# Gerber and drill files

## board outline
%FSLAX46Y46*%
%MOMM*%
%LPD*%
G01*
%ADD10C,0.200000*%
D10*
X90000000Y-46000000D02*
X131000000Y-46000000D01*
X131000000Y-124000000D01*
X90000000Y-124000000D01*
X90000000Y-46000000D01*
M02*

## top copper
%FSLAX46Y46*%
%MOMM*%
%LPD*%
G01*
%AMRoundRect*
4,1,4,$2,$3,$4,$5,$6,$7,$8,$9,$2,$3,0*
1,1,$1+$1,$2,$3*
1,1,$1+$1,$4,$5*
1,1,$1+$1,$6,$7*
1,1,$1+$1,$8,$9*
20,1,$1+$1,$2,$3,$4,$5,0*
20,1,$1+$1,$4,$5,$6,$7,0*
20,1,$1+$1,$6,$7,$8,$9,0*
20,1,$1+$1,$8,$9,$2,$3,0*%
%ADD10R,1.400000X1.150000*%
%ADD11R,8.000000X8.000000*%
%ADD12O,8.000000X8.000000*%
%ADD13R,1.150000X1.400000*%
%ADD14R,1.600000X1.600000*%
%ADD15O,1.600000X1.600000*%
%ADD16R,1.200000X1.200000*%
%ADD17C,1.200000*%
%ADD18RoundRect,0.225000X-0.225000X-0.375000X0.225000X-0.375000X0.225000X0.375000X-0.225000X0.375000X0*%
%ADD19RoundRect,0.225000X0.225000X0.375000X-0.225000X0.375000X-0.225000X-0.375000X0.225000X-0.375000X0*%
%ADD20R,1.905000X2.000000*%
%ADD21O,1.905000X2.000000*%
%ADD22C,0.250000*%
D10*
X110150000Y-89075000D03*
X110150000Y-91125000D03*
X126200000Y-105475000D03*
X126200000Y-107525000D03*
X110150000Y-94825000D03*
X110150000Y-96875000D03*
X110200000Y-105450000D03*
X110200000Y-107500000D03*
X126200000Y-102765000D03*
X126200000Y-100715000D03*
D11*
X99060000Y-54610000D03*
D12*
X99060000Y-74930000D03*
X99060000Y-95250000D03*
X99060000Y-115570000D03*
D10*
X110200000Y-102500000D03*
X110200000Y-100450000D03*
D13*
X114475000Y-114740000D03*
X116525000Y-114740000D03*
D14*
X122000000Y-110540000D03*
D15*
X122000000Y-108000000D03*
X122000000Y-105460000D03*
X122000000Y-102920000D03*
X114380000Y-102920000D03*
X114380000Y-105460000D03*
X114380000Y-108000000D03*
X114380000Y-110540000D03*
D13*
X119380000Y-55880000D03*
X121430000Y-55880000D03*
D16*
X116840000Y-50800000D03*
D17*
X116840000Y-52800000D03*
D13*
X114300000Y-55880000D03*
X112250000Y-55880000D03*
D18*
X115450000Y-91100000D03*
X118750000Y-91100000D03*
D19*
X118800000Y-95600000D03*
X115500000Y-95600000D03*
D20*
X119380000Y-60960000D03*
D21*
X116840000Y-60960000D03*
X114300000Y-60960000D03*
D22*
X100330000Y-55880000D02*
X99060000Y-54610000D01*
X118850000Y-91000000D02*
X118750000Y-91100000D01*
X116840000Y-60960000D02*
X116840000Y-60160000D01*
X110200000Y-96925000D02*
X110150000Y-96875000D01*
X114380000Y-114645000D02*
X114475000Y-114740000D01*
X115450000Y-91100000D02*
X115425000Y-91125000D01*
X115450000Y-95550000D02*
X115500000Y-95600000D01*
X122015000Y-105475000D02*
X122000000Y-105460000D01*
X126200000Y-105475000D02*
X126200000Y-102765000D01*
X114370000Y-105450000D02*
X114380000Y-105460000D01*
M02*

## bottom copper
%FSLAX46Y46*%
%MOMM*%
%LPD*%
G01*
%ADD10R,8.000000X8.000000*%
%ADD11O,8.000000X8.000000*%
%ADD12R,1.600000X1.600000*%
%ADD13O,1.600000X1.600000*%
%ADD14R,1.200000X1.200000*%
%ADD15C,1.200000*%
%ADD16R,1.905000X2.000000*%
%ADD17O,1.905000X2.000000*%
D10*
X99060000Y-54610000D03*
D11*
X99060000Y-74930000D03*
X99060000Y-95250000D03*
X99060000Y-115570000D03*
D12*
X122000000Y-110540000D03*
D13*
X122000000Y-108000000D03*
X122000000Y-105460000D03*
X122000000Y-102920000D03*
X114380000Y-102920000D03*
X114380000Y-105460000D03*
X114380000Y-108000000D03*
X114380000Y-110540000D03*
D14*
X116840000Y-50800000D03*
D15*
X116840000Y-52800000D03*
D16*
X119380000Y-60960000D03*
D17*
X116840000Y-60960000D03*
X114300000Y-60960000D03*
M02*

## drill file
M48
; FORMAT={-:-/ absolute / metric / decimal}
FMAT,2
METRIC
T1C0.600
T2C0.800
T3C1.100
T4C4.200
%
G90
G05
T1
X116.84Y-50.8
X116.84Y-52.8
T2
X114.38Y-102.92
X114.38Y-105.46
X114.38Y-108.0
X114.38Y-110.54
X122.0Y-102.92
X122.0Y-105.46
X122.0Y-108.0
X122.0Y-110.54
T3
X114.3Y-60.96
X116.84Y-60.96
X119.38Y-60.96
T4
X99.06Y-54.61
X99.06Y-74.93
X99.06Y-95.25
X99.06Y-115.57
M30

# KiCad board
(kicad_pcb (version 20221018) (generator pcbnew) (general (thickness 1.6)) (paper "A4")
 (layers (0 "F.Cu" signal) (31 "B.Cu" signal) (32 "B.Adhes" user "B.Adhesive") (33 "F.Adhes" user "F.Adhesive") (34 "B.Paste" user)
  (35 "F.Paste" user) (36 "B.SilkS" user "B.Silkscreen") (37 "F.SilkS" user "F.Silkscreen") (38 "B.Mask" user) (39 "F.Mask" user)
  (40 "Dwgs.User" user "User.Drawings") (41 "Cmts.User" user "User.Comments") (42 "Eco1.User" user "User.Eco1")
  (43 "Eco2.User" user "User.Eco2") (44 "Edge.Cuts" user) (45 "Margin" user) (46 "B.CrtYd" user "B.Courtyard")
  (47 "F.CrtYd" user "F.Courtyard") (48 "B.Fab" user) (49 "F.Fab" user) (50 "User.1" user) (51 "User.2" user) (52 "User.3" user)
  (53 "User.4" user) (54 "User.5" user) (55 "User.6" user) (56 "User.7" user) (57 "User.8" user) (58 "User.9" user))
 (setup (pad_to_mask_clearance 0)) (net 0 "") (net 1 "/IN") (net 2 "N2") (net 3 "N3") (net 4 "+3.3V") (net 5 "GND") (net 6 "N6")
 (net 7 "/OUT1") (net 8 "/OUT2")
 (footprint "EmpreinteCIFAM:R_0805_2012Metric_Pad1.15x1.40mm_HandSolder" (layer "F.Cu") (at 110.15 90.1 -90)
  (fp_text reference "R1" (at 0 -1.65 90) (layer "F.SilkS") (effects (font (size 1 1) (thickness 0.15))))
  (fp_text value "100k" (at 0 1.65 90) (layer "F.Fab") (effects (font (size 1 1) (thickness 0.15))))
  (pad "1" smd rect (at -1.025 0 270) (size 1.15 1.4) (layers "F.Cu" "F.Paste" "F.Mask") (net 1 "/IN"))
  (pad "2" smd rect (at 1.025 0 270) (size 1.15 1.4) (layers "F.Cu" "F.Paste" "F.Mask") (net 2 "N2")))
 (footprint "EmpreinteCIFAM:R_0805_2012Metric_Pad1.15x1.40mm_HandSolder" (layer "F.Cu") (at 126.2 106.5 -90)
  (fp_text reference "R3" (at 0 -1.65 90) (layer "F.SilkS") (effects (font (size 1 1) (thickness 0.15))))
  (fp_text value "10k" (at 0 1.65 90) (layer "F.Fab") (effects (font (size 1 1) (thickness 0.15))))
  (pad "1" smd rect (at -1.025 0 270) (size 1.15 1.4) (layers "F.Cu" "F.Paste" "F.Mask") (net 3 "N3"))
  (pad "2" smd rect (at 1.025 0 270) (size 1.15 1.4) (layers "F.Cu" "F.Paste" "F.Mask") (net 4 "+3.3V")))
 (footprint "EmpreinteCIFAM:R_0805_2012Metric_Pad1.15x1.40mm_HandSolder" (layer "F.Cu") (at 110.15 95.85 -90)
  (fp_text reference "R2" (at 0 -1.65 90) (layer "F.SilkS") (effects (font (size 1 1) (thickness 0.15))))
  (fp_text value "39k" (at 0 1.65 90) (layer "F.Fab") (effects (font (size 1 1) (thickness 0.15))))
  (pad "1" smd rect (at -1.025 0 270) (size 1.15 1.4) (layers "F.Cu" "F.Paste" "F.Mask") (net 2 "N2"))
  (pad "2" smd rect (at 1.025 0 270) (size 1.15 1.4) (layers "F.Cu" "F.Paste" "F.Mask") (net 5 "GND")))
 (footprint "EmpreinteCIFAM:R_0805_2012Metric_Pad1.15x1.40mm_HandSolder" (layer "F.Cu") (at 110.2 106.475 -90)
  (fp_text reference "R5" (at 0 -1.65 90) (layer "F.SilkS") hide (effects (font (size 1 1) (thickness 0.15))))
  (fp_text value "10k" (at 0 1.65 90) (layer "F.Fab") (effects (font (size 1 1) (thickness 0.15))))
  (pad "1" smd rect (at -1.025 0 270) (size 1.15 1.4) (layers "F.Cu" "F.Paste" "F.Mask") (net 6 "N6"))
  (pad "2" smd rect (at 1.025 0 270) (size 1.15 1.4) (layers "F.Cu" "F.Paste" "F.Mask") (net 4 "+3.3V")))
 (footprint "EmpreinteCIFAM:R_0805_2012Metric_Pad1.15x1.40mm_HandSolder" (layer "F.Cu") (at 126.2 101.74 90)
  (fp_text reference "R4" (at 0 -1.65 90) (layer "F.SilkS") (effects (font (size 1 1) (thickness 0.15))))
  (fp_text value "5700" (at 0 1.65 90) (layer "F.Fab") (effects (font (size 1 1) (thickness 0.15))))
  (pad "1" smd rect (at -1.025 0 90) (size 1.15 1.4) (layers "F.Cu" "F.Paste" "F.Mask") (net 3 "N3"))
  (pad "2" smd rect (at 1.025 0 90) (size 1.15 1.4) (layers "F.Cu" "F.Paste" "F.Mask") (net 5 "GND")))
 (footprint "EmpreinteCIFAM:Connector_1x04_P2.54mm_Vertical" (layer "F.Cu") (at 124.46 68.58)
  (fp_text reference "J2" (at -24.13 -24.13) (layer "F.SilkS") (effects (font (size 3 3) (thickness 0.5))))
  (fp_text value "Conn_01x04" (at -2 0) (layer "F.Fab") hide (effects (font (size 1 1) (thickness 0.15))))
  (pad "1" thru_hole rect (at -25.4 -13.97) (size 8 8) (drill 4.2) (layers "*.Cu" "*.Mask") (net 1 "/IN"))
  (pad "2" thru_hole oval (at -25.4 6.35) (size 8 8) (drill 4.2) (layers "*.Cu" "*.Mask") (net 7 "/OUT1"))
  (pad "3" thru_hole oval (at -25.4 26.67) (size 8 8) (drill 4.2) (layers "*.Cu" "*.Mask") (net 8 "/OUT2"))
  (pad "4" thru_hole oval (at -25.4 46.99) (size 8 8) (drill 4.2) (layers "*.Cu" "*.Mask") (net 5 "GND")))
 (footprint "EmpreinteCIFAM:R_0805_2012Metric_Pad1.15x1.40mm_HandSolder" (layer "F.Cu") (at 110.2 101.475 90)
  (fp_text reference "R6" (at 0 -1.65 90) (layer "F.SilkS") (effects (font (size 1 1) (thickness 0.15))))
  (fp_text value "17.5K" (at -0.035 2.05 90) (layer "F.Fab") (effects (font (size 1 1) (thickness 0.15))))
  (pad "1" smd rect (at -1.025 0 90) (size 1.15 1.4) (layers "F.Cu" "F.Paste" "F.Mask") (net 6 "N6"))
  (pad "2" smd rect (at 1.025 0 90) (size 1.15 1.4) (layers "F.Cu" "F.Paste" "F.Mask") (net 5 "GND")))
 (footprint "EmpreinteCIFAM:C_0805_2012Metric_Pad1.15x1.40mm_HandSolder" (layer "F.Cu") (at 115.5 114.74)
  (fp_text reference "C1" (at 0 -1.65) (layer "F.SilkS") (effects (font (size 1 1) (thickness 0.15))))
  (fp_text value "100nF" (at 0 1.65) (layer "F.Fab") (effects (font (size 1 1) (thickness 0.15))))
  (pad "1" smd rect (at -1.025 0) (size 1.15 1.4) (layers "F.Cu" "F.Paste" "F.Mask") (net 4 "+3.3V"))
  (pad "2" smd rect (at 1.025 0) (size 1.15 1.4) (layers "F.Cu" "F.Paste" "F.Mask") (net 5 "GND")))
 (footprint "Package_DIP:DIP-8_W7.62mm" (layer "F.Cu") (at 122 110.54 180)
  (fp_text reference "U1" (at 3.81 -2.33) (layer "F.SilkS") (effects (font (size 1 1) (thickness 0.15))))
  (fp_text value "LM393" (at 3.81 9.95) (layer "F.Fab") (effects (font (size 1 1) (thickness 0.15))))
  (pad "1" thru_hole rect (at 0 0 180) (size 1.6 1.6) (drill 0.8) (layers "*.Cu" "*.Mask") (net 7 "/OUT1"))
  (pad "2" thru_hole oval (at 0 2.54 180) (size 1.6 1.6) (drill 0.8) (layers "*.Cu" "*.Mask") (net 2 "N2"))
  (pad "3" thru_hole oval (at 0 5.08 180) (size 1.6 1.6) (drill 0.8) (layers "*.Cu" "*.Mask") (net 3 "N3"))
  (pad "4" thru_hole oval (at 0 7.62 180) (size 1.6 1.6) (drill 0.8) (layers "*.Cu" "*.Mask") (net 5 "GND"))
  (pad "5" thru_hole oval (at 7.62 7.62 180) (size 1.6 1.6) (drill 0.8) (layers "*.Cu" "*.Mask") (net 2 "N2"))
  (pad "6" thru_hole oval (at 7.62 5.08 180) (size 1.6 1.6) (drill 0.8) (layers "*.Cu" "*.Mask") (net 6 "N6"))
  (pad "7" thru_hole oval (at 7.62 2.54 180) (size 1.6 1.6) (drill 0.8) (layers "*.Cu" "*.Mask") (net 8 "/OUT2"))
  (pad "8" thru_hole oval (at 7.62 0 180) (size 1.6 1.6) (drill 0.8) (layers "*.Cu" "*.Mask") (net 4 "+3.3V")))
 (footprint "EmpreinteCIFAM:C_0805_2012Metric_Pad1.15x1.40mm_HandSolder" (layer "F.Cu") (at 120.405 55.88)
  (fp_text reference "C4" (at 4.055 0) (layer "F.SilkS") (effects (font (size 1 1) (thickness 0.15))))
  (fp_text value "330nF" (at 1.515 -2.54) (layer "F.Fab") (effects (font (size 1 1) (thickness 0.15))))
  (pad "1" smd rect (at -1.025 0) (size 1.15 1.4) (layers "F.Cu" "F.Paste" "F.Mask") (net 5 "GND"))
  (pad "2" smd rect (at 1.025 0) (size 1.15 1.4) (layers "F.Cu" "F.Paste" "F.Mask") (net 4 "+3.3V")))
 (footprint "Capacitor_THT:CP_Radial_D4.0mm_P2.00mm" (layer "F.Cu") (at 116.84 50.8 -90)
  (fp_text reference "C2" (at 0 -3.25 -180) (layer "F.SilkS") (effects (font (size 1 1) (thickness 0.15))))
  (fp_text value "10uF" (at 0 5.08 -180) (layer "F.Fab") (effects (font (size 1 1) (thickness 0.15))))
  (pad "1" thru_hole rect (at 0 0 270) (size 1.2 1.2) (drill 0.6) (layers "*.Cu" "*.Mask") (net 1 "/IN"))
  (pad "2" thru_hole circle (at 2 0 270) (size 1.2 1.2) (drill 0.6) (layers "*.Cu" "*.Mask") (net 5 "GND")))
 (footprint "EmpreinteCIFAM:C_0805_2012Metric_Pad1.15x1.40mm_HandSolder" (layer "F.Cu") (at 113.275 55.88 180)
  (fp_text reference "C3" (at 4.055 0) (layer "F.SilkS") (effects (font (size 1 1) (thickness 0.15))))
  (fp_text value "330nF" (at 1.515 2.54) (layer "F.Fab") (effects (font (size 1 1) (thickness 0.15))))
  (pad "1" smd rect (at -1.025 0 180) (size 1.15 1.4) (layers "F.Cu" "F.Paste" "F.Mask") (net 5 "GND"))
  (pad "2" smd rect (at 1.025 0 180) (size 1.15 1.4) (layers "F.Cu" "F.Paste" "F.Mask") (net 1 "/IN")))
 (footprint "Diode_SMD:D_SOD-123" (layer "F.Cu") (at 117.1 91.1)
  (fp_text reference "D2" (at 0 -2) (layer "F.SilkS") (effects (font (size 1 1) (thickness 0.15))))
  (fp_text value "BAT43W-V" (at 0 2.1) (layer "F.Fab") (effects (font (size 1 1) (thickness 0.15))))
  (pad "1" smd roundrect (at -1.65 0) (size 0.9 1.2) (layers "F.Cu" "F.Paste" "F.Mask") (roundrect_rratio 0.25) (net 2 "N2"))
  (pad "2" smd roundrect (at 1.65 0) (size 0.9 1.2) (layers "F.Cu" "F.Paste" "F.Mask") (roundrect_rratio 0.25) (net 5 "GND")))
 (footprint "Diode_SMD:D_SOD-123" (layer "F.Cu") (at 117.15 95.6 180)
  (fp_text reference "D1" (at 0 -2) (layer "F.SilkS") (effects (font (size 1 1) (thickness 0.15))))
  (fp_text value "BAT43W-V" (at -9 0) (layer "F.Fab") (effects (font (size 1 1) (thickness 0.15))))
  (pad "1" smd roundrect (at -1.65 0 180) (size 0.9 1.2) (layers "F.Cu" "F.Paste" "F.Mask") (roundrect_rratio 0.25) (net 4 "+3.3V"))
  (pad "2" smd roundrect (at 1.65 0 180) (size 0.9 1.2) (layers "F.Cu" "F.Paste" "F.Mask") (roundrect_rratio 0.25) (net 2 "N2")))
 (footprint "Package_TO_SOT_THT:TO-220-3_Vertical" (layer "F.Cu") (at 119.38 60.96 180)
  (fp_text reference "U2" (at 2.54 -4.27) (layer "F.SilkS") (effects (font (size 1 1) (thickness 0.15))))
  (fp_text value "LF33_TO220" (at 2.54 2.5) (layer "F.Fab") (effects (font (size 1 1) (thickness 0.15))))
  (pad "1" thru_hole rect (at 0 0 180) (size 1.905 2) (drill 1.1) (layers "*.Cu" "*.Mask") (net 1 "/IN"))
  (pad "2" thru_hole oval (at 2.54 0 180) (size 1.905 2) (drill 1.1) (layers "*.Cu" "*.Mask") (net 5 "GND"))
  (pad "3" thru_hole oval (at 5.08 0 180) (size 1.905 2) (drill 1.1) (layers "*.Cu" "*.Mask") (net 4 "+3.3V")))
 (gr_rect (start 90 46) (end 131 124) (stroke (width 0.2) (type default)) (fill none) (layer "Edge.Cuts"))
 (segment (start 100.33 55.88) (end 99.06 54.61) (width 0.25) (layer "F.Cu") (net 1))
 (segment (start 118.85 91) (end 118.75 91.1) (width 0.25) (layer "F.Cu") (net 5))
 (segment (start 116.84 60.96) (end 116.84 60.16) (width 0.25) (layer "F.Cu") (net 5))
 (segment (start 110.2 96.925) (end 110.15 96.875) (width 0.25) (layer "F.Cu") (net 5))
 (segment (start 114.38 114.645) (end 114.475 114.74) (width 0.25) (layer "F.Cu") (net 4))
 (segment (start 115.45 91.1) (end 115.425 91.125) (width 0.25) (layer "F.Cu") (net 2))
 (segment (start 115.45 95.55) (end 115.5 95.6) (width 0.25) (layer "F.Cu") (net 2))
 (segment (start 122.015 105.475) (end 122 105.46) (width 0.25) (layer "F.Cu") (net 3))
 (segment (start 126.2 105.475) (end 126.2 102.765) (width 0.25) (layer "F.Cu") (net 3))
 (segment (start 114.37 105.45) (end 114.38 105.46) (width 0.25) (layer "F.Cu") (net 6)))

